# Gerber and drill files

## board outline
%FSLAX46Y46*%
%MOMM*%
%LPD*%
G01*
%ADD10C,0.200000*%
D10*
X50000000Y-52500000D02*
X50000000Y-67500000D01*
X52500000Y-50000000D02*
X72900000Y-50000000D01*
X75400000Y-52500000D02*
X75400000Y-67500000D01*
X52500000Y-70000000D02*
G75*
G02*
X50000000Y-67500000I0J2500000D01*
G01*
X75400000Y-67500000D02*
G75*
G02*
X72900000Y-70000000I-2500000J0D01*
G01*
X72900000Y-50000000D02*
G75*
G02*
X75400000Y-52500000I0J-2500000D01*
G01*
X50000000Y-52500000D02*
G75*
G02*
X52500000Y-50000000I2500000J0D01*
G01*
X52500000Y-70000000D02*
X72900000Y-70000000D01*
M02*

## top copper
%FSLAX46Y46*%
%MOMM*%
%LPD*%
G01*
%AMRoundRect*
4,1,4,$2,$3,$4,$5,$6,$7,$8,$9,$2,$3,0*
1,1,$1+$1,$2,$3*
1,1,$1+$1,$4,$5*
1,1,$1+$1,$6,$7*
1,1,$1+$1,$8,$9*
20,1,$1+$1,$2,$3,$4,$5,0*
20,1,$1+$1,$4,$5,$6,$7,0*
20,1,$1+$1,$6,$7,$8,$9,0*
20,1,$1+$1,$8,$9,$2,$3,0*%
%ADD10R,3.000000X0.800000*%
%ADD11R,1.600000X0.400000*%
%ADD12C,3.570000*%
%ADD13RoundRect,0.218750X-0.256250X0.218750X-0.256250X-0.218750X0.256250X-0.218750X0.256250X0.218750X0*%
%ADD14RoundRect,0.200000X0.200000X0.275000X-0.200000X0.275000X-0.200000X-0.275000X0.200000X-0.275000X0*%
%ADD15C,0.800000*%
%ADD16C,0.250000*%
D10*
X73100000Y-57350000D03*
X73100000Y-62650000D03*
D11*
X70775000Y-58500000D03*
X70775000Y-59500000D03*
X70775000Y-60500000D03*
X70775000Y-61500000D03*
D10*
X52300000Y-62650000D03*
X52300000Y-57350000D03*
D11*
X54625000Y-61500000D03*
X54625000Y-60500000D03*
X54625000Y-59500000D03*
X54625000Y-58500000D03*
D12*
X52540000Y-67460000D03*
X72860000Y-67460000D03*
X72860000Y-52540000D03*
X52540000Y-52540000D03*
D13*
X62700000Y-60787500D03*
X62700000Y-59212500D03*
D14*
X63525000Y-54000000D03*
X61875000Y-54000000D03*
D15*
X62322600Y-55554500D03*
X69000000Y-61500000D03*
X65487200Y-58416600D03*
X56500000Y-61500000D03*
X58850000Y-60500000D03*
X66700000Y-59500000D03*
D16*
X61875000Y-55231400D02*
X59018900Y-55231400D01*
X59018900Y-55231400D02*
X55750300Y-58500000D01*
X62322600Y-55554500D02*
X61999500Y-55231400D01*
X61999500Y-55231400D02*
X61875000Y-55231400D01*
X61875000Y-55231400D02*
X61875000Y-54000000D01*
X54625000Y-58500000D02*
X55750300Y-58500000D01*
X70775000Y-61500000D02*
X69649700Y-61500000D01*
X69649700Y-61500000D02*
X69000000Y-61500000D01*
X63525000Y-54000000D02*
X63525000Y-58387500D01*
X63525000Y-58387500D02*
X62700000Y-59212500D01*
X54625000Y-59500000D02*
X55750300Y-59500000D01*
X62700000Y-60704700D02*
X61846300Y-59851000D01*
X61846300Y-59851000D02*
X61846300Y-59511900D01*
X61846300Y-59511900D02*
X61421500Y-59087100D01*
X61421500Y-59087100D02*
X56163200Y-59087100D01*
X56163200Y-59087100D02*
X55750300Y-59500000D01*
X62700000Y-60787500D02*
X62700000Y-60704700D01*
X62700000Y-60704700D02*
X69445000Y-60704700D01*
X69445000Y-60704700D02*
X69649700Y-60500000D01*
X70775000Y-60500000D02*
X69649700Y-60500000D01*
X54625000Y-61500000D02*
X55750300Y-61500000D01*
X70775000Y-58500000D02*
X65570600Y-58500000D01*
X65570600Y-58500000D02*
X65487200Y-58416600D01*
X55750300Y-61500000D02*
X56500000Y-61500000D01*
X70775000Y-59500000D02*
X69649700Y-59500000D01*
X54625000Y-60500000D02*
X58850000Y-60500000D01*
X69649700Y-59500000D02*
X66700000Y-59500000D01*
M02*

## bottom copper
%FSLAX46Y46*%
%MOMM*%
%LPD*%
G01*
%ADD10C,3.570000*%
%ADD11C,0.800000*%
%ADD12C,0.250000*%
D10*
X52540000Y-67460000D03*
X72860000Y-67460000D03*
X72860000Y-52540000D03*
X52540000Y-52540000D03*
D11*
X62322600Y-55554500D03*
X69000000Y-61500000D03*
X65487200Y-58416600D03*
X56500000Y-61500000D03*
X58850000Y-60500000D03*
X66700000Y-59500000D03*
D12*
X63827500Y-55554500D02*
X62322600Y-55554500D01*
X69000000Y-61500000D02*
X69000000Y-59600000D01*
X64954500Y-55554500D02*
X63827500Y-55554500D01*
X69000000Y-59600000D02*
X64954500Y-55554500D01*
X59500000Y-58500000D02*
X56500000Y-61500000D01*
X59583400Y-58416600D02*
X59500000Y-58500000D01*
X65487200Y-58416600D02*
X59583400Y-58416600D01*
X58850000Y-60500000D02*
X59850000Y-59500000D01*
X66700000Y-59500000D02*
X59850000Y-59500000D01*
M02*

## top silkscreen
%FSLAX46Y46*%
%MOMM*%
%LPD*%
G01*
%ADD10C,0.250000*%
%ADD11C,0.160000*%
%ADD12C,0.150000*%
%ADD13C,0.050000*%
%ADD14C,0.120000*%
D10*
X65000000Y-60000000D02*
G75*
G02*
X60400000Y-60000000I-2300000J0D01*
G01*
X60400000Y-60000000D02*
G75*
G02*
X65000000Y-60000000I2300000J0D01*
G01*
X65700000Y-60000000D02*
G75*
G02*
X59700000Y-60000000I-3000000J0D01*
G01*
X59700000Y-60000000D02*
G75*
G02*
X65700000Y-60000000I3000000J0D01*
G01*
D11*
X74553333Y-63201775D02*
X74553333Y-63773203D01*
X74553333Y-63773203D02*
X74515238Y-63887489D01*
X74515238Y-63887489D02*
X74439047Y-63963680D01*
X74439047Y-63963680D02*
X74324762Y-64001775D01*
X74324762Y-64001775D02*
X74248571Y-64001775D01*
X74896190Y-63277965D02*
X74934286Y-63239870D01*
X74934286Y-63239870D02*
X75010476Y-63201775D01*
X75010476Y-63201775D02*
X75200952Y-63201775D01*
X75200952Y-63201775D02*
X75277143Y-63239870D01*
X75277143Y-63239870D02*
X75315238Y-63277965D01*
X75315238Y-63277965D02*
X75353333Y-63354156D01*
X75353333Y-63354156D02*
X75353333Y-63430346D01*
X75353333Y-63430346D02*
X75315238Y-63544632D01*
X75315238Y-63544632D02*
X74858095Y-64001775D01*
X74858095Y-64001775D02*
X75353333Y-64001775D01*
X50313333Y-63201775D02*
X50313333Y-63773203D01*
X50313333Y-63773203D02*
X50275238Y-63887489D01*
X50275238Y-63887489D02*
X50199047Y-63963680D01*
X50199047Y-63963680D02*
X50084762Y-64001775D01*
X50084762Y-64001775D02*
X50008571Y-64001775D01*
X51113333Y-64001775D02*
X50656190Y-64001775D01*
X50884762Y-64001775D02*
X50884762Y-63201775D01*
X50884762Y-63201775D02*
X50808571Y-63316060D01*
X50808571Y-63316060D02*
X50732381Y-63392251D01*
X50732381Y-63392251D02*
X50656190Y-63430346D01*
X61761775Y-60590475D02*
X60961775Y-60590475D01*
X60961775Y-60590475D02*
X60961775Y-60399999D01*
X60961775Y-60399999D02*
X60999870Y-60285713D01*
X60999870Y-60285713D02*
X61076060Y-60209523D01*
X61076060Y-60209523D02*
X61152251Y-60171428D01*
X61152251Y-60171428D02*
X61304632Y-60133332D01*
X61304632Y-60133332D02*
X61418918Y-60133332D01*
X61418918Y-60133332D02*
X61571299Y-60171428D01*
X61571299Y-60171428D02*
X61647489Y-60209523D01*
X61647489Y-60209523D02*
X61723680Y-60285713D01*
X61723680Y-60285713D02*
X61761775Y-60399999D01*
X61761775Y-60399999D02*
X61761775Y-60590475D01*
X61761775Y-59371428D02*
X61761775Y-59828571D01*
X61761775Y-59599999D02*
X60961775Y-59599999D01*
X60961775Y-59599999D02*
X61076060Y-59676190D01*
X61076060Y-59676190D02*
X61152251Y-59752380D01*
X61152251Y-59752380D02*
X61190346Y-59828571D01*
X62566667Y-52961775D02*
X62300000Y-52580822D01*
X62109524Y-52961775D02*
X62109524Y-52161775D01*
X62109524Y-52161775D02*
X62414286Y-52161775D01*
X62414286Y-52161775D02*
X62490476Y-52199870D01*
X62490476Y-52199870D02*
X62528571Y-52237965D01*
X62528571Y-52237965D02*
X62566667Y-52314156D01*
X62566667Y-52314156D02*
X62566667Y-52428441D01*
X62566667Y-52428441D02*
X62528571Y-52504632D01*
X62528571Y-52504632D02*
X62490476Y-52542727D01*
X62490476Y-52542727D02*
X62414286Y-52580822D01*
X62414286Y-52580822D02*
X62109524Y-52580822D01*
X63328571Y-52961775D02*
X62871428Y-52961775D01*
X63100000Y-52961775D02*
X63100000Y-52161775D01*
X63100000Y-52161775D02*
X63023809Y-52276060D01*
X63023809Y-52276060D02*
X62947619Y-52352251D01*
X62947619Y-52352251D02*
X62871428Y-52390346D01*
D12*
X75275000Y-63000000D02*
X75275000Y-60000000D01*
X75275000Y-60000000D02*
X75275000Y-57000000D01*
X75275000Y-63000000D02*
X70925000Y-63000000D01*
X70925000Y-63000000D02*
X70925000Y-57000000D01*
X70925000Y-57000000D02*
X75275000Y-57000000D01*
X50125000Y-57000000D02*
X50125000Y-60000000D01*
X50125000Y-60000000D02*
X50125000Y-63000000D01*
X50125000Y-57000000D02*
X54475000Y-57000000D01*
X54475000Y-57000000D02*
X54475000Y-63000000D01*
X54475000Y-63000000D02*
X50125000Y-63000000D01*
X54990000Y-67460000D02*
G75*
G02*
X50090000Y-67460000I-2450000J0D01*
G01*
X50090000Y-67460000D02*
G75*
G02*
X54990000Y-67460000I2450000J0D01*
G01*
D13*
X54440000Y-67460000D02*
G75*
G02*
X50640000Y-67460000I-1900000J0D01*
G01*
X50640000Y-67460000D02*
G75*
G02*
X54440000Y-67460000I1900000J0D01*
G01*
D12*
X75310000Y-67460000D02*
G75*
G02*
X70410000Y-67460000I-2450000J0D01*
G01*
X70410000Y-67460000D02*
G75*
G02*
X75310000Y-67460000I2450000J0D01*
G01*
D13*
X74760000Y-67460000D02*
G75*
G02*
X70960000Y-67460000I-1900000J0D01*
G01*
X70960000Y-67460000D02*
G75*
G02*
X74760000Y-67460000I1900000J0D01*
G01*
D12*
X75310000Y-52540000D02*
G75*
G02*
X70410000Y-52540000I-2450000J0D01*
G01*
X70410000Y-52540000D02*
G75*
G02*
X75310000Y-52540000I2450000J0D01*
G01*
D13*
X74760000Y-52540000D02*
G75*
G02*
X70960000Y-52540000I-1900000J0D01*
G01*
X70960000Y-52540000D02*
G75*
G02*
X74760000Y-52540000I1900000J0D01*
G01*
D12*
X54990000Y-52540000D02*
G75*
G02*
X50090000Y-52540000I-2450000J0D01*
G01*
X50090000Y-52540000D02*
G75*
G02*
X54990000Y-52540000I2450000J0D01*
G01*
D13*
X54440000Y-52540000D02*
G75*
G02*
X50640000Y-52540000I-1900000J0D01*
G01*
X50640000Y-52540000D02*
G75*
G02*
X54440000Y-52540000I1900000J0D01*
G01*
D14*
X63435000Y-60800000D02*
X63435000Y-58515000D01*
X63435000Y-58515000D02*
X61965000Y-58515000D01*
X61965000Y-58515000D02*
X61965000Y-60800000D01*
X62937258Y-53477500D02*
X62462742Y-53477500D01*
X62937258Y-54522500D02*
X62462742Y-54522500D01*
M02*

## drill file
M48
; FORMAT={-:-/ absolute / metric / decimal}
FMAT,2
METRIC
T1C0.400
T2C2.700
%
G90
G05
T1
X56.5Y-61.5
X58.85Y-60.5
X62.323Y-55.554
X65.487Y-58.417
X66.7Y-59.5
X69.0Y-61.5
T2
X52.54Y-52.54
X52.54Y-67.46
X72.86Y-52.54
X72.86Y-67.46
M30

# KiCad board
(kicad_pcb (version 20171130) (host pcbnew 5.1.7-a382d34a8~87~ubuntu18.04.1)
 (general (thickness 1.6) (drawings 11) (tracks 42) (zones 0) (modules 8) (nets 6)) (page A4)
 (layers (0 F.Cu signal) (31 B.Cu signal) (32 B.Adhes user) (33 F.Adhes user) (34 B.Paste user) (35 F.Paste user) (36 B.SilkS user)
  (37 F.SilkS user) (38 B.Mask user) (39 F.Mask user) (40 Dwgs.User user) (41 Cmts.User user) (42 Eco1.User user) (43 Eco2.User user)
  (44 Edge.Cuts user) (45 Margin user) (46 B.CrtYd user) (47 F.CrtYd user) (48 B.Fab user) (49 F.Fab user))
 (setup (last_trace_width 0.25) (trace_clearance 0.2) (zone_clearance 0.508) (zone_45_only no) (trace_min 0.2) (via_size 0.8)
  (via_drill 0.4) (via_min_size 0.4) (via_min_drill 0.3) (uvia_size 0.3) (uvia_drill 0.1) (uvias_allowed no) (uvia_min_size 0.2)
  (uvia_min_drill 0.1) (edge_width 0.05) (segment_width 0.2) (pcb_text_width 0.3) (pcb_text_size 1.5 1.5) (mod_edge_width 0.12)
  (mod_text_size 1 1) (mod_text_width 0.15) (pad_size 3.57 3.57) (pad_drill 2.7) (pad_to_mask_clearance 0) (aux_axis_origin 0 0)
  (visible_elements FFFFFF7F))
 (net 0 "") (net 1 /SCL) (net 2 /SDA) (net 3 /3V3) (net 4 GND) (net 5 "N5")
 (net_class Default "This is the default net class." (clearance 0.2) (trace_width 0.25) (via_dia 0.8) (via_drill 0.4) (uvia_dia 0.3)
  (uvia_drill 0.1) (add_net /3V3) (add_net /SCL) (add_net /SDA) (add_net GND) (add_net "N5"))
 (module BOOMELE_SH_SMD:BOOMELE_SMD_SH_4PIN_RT (layer F.Cu) (at 72.62 60 270)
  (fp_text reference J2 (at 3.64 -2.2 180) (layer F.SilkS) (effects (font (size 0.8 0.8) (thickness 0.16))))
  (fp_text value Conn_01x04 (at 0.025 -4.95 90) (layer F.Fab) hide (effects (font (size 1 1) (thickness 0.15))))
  (fp_line (start 3 -2.655) (end 0 -2.655) (layer F.SilkS) (width 0.15))
  (fp_line (start 0 -2.655) (end -3 -2.655) (layer F.SilkS) (width 0.15))
  (fp_line (start 3 -2.655) (end 3 1.695) (layer F.SilkS) (width 0.15))
  (fp_line (start 3 1.695) (end -3 1.695) (layer F.SilkS) (width 0.15))
  (fp_line (start -3 1.695) (end -3 -2.655) (layer F.SilkS) (width 0.15))
  (pad "" smd rect (at -2.65 -0.48 90) (size 0.8 3) (layers F.Cu F.Paste F.Mask))
  (pad "" smd rect (at 2.65 -0.48 90) (size 0.8 3) (layers F.Cu F.Paste F.Mask))
  (pad 4 smd rect (at -1.5 1.845 90) (size 0.4 1.6) (layers F.Cu F.Paste F.Mask) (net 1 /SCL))
  (pad 3 smd rect (at -0.5 1.845 90) (size 0.4 1.6) (layers F.Cu F.Paste F.Mask) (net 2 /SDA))
  (pad 2 smd rect (at 0.5 1.845 90) (size 0.4 1.6) (layers F.Cu F.Paste F.Mask) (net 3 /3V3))
  (pad 1 smd rect (at 1.5 1.845 90) (size 0.4 1.6) (layers F.Cu F.Paste F.Mask) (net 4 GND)))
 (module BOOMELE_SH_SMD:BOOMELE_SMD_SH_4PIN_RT (layer F.Cu) (at 52.78 60 90)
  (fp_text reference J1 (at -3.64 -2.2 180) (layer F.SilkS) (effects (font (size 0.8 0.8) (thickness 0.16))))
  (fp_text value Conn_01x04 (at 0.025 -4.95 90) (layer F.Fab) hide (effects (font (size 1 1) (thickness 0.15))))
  (fp_line (start 3 -2.655) (end 0 -2.655) (layer F.SilkS) (width 0.15))
  (fp_line (start 0 -2.655) (end -3 -2.655) (layer F.SilkS) (width 0.15))
  (fp_line (start 3 -2.655) (end 3 1.695) (layer F.SilkS) (width 0.15))
  (fp_line (start 3 1.695) (end -3 1.695) (layer F.SilkS) (width 0.15))
  (fp_line (start -3 1.695) (end -3 -2.655) (layer F.SilkS) (width 0.15))
  (pad "" smd rect (at -2.65 -0.48 270) (size 0.8 3) (layers F.Cu F.Paste F.Mask))
  (pad "" smd rect (at 2.65 -0.48 270) (size 0.8 3) (layers F.Cu F.Paste F.Mask))
  (pad 4 smd rect (at -1.5 1.845 270) (size 0.4 1.6) (layers F.Cu F.Paste F.Mask) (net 1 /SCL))
  (pad 3 smd rect (at -0.5 1.845 270) (size 0.4 1.6) (layers F.Cu F.Paste F.Mask) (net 2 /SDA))
  (pad 2 smd rect (at 0.5 1.845 270) (size 0.4 1.6) (layers F.Cu F.Paste F.Mask) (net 3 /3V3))
  (pad 1 smd rect (at 1.5 1.845 270) (size 0.4 1.6) (layers F.Cu F.Paste F.Mask) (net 4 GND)))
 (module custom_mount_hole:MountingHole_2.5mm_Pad (layer F.Cu) (at 52.54 67.46)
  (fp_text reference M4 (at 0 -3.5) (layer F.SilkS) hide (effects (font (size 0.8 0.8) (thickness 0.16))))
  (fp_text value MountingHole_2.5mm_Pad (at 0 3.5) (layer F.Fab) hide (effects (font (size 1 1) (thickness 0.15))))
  (fp_circle (center 0 0) (end 2.45 0) (layer F.SilkS) (width 0.15))
  (fp_circle (center 0 0) (end 1.9 0) (layer F.SilkS) (width 0.05))
  (pad ~ thru_hole circle (at 0 0) (size 3.57 3.57) (drill 2.7) (layers *.Cu *.Mask)))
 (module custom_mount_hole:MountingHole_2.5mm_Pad (layer F.Cu) (at 72.86 67.46)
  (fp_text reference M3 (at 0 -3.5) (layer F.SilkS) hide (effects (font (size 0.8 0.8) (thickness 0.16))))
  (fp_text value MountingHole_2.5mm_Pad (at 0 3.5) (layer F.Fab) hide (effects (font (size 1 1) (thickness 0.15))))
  (fp_circle (center 0 0) (end 2.45 0) (layer F.SilkS) (width 0.15))
  (fp_circle (center 0 0) (end 1.9 0) (layer F.SilkS) (width 0.05))
  (pad ~ thru_hole circle (at 0 0) (size 3.57 3.57) (drill 2.7) (layers *.Cu *.Mask)))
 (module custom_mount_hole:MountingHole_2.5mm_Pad (layer F.Cu) (at 72.86 52.54)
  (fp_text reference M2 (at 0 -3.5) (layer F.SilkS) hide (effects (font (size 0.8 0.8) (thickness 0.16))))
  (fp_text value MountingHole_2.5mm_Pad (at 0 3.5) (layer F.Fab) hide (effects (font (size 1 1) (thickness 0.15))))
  (fp_circle (center 0 0) (end 2.45 0) (layer F.SilkS) (width 0.15))
  (fp_circle (center 0 0) (end 1.9 0) (layer F.SilkS) (width 0.05))
  (pad ~ thru_hole circle (at 0 0) (size 3.57 3.57) (drill 2.7) (layers *.Cu *.Mask)))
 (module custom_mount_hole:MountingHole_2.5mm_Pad (layer F.Cu) (at 52.54 52.54)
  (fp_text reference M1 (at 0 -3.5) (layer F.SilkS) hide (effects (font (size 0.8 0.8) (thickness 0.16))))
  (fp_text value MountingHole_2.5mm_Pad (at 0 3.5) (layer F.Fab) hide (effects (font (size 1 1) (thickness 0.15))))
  (fp_circle (center 0 0) (end 2.45 0) (layer F.SilkS) (width 0.15))
  (fp_circle (center 0 0) (end 1.9 0) (layer F.SilkS) (width 0.05))
  (pad ~ thru_hole circle (at 0 0) (size 3.57 3.57) (drill 2.7) (layers *.Cu *.Mask)))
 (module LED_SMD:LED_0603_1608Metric (layer F.Cu) (at 62.7 60 270)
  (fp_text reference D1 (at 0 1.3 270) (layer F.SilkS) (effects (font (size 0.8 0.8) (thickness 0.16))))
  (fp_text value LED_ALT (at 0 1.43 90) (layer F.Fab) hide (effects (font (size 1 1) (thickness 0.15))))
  (fp_line (start 0.8 -0.735) (end -1.485 -0.735) (layer F.SilkS) (width 0.12))
  (fp_line (start -1.485 -0.735) (end -1.485 0.735) (layer F.SilkS) (width 0.12))
  (fp_line (start -1.485 0.735) (end 0.8 0.735) (layer F.SilkS) (width 0.12))
  (pad 2 smd roundrect (at 0.7875 0 270) (size 0.875 0.95) (layers F.Cu F.Paste F.Mask) (roundrect_rratio 0.25) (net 3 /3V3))
  (pad 1 smd roundrect (at -0.7875 0 270) (size 0.875 0.95) (layers F.Cu F.Paste F.Mask) (roundrect_rratio 0.25) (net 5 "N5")))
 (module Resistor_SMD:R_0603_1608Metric (layer F.Cu) (at 62.7 54 180)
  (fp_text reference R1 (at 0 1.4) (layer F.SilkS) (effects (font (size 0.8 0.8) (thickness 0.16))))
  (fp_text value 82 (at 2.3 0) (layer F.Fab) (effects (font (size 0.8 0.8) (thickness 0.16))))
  (fp_line (start -0.237258 0.5225) (end 0.237258 0.5225) (layer F.SilkS) (width 0.12))
  (fp_line (start -0.237258 -0.5225) (end 0.237258 -0.5225) (layer F.SilkS) (width 0.12))
  (pad 1 smd roundrect (at -0.825 0 180) (size 0.8 0.95) (layers F.Cu F.Paste F.Mask) (roundrect_rratio 0.25) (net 5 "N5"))
  (pad 2 smd roundrect (at 0.825 0 180) (size 0.8 0.95) (layers F.Cu F.Paste F.Mask) (roundrect_rratio 0.25) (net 4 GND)))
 (gr_circle (center 62.7 60) (end 65 60) (layer F.SilkS) (width 0.25))
 (gr_circle (center 62.7 60) (end 65.7 60) (layer F.SilkS) (width 0.25))
 (gr_line (start 50 52.5) (end 50 67.5) (layer Edge.Cuts) (width 0.2))
 (gr_line (start 52.5 50) (end 72.9 50) (layer Edge.Cuts) (width 0.2))
 (gr_line (start 75.4 52.5) (end 75.4 67.5) (layer Edge.Cuts) (width 0.2))
 (gr_arc (start 52.5 67.5) (end 50 67.5) (angle -90) (layer Edge.Cuts) (width 0.2))
 (gr_arc (start 72.9 67.5) (end 72.9 70) (angle -90) (layer Edge.Cuts) (width 0.2))
 (gr_arc (start 72.9 52.5) (end 75.4 52.5) (angle -90) (layer Edge.Cuts) (width 0.2))
 (gr_arc (start 52.5 52.5) (end 52.5 50) (angle -90) (layer Edge.Cuts) (width 0.2))
 (gr_line (start 52.5 70) (end 72.9 70) (layer Edge.Cuts) (width 0.2))
 (segment (start 63.8275 55.5545) (end 62.3226 55.5545) (width 0.25) (layer B.Cu) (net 4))
 (segment (start 61.875 55.2314) (end 59.0189 55.2314) (width 0.25) (layer F.Cu) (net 4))
 (segment (start 59.0189 55.2314) (end 55.7503 58.5) (width 0.25) (layer F.Cu) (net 4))
 (segment (start 62.3226 55.5545) (end 61.9995 55.2314) (width 0.25) (layer F.Cu) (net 4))
 (segment (start 61.9995 55.2314) (end 61.875 55.2314) (width 0.25) (layer F.Cu) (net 4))
 (segment (start 61.875 55.2314) (end 61.875 54) (width 0.25) (layer F.Cu) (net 4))
 (segment (start 54.625 58.5) (end 55.7503 58.5) (width 0.25) (layer F.Cu) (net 4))
 (segment (start 70.775 61.5) (end 69.6497 61.5) (width 0.25) (layer F.Cu) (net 4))
 (via (at 62.3226 55.5545) (size 0.8) (layers F.Cu B.Cu) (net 4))
 (via (at 69 61.5) (size 0.8) (drill 0.4) (layers F.Cu B.Cu) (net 4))
 (segment (start 69.6497 61.5) (end 69 61.5) (width 0.25) (layer F.Cu) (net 4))
 (segment (start 69 61.5) (end 69 59.6) (width 0.25) (layer B.Cu) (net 4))
 (segment (start 64.9545 55.5545) (end 63.8275 55.5545) (width 0.25) (layer B.Cu) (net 4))
 (segment (start 69 59.6) (end 64.9545 55.5545) (width 0.25) (layer B.Cu) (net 4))
 (segment (start 63.525 54) (end 63.525 58.3875) (width 0.25) (layer F.Cu) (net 5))
 (segment (start 63.525 58.3875) (end 62.7 59.2125) (width 0.25) (layer F.Cu) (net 5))
 (segment (start 54.625 59.5) (end 55.7503 59.5) (width 0.25) (layer F.Cu) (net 3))
 (segment (start 62.7 60.7047) (end 61.8463 59.851) (width 0.25) (layer F.Cu) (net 3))
 (segment (start 61.8463 59.851) (end 61.8463 59.5119) (width 0.25) (layer F.Cu) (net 3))
 (segment (start 61.8463 59.5119) (end 61.4215 59.0871) (width 0.25) (layer F.Cu) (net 3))
 (segment (start 61.4215 59.0871) (end 56.1632 59.0871) (width 0.25) (layer F.Cu) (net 3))
 (segment (start 56.1632 59.0871) (end 55.7503 59.5) (width 0.25) (layer F.Cu) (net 3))
 (segment (start 62.7 60.7875) (end 62.7 60.7047) (width 0.25) (layer F.Cu) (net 3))
 (segment (start 62.7 60.7047) (end 69.445 60.7047) (width 0.25) (layer F.Cu) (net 3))
 (segment (start 69.445 60.7047) (end 69.6497 60.5) (width 0.25) (layer F.Cu) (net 3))
 (segment (start 70.775 60.5) (end 69.6497 60.5) (width 0.25) (layer F.Cu) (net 3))
 (segment (start 54.625 61.5) (end 55.7503 61.5) (width 0.25) (layer F.Cu) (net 1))
 (segment (start 70.775 58.5) (end 65.5706 58.5) (width 0.25) (layer F.Cu) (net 1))
 (segment (start 65.5706 58.5) (end 65.4872 58.4166) (width 0.25) (layer F.Cu) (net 1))
 (via (at 65.4872 58.4166) (size 0.8) (layers F.Cu B.Cu) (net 1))
 (via (at 56.5 61.5) (size 0.8) (drill 0.4) (layers F.Cu B.Cu) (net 1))
 (segment (start 55.7503 61.5) (end 56.5 61.5) (width 0.25) (layer F.Cu) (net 1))
 (segment (start 59.5 58.5) (end 56.5 61.5) (width 0.25) (layer B.Cu) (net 1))
 (segment (start 59.5834 58.4166) (end 59.5 58.5) (width 0.25) (layer B.Cu) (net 1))
 (segment (start 65.4872 58.4166) (end 59.5834 58.4166) (width 0.25) (layer B.Cu) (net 1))
 (segment (start 70.775 59.5) (end 69.6497 59.5) (width 0.25) (layer F.Cu) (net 2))
 (via (at 58.85 60.5) (size 0.8) (drill 0.4) (layers F.Cu B.Cu) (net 2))
 (segment (start 54.625 60.5) (end 58.85 60.5) (width 0.25) (layer F.Cu) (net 2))
 (segment (start 58.85 60.5) (end 59.85 59.5) (width 0.25) (layer B.Cu) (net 2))
 (via (at 66.7 59.5) (size 0.8) (drill 0.4) (layers F.Cu B.Cu) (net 2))
 (segment (start 69.6497 59.5) (end 66.7 59.5) (width 0.25) (layer F.Cu) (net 2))
 (segment (start 66.7 59.5) (end 59.85 59.5) (width 0.25) (layer B.Cu) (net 2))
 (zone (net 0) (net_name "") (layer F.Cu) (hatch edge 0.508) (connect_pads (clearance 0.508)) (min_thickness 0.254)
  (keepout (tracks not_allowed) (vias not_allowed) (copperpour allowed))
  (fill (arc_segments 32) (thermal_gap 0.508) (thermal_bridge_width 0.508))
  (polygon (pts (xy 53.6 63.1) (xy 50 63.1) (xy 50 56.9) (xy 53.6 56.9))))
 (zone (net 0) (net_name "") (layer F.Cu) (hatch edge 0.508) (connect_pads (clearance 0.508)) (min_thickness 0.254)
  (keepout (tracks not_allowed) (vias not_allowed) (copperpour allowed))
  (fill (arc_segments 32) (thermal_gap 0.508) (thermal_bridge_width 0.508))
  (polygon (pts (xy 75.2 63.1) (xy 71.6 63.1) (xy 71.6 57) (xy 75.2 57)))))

